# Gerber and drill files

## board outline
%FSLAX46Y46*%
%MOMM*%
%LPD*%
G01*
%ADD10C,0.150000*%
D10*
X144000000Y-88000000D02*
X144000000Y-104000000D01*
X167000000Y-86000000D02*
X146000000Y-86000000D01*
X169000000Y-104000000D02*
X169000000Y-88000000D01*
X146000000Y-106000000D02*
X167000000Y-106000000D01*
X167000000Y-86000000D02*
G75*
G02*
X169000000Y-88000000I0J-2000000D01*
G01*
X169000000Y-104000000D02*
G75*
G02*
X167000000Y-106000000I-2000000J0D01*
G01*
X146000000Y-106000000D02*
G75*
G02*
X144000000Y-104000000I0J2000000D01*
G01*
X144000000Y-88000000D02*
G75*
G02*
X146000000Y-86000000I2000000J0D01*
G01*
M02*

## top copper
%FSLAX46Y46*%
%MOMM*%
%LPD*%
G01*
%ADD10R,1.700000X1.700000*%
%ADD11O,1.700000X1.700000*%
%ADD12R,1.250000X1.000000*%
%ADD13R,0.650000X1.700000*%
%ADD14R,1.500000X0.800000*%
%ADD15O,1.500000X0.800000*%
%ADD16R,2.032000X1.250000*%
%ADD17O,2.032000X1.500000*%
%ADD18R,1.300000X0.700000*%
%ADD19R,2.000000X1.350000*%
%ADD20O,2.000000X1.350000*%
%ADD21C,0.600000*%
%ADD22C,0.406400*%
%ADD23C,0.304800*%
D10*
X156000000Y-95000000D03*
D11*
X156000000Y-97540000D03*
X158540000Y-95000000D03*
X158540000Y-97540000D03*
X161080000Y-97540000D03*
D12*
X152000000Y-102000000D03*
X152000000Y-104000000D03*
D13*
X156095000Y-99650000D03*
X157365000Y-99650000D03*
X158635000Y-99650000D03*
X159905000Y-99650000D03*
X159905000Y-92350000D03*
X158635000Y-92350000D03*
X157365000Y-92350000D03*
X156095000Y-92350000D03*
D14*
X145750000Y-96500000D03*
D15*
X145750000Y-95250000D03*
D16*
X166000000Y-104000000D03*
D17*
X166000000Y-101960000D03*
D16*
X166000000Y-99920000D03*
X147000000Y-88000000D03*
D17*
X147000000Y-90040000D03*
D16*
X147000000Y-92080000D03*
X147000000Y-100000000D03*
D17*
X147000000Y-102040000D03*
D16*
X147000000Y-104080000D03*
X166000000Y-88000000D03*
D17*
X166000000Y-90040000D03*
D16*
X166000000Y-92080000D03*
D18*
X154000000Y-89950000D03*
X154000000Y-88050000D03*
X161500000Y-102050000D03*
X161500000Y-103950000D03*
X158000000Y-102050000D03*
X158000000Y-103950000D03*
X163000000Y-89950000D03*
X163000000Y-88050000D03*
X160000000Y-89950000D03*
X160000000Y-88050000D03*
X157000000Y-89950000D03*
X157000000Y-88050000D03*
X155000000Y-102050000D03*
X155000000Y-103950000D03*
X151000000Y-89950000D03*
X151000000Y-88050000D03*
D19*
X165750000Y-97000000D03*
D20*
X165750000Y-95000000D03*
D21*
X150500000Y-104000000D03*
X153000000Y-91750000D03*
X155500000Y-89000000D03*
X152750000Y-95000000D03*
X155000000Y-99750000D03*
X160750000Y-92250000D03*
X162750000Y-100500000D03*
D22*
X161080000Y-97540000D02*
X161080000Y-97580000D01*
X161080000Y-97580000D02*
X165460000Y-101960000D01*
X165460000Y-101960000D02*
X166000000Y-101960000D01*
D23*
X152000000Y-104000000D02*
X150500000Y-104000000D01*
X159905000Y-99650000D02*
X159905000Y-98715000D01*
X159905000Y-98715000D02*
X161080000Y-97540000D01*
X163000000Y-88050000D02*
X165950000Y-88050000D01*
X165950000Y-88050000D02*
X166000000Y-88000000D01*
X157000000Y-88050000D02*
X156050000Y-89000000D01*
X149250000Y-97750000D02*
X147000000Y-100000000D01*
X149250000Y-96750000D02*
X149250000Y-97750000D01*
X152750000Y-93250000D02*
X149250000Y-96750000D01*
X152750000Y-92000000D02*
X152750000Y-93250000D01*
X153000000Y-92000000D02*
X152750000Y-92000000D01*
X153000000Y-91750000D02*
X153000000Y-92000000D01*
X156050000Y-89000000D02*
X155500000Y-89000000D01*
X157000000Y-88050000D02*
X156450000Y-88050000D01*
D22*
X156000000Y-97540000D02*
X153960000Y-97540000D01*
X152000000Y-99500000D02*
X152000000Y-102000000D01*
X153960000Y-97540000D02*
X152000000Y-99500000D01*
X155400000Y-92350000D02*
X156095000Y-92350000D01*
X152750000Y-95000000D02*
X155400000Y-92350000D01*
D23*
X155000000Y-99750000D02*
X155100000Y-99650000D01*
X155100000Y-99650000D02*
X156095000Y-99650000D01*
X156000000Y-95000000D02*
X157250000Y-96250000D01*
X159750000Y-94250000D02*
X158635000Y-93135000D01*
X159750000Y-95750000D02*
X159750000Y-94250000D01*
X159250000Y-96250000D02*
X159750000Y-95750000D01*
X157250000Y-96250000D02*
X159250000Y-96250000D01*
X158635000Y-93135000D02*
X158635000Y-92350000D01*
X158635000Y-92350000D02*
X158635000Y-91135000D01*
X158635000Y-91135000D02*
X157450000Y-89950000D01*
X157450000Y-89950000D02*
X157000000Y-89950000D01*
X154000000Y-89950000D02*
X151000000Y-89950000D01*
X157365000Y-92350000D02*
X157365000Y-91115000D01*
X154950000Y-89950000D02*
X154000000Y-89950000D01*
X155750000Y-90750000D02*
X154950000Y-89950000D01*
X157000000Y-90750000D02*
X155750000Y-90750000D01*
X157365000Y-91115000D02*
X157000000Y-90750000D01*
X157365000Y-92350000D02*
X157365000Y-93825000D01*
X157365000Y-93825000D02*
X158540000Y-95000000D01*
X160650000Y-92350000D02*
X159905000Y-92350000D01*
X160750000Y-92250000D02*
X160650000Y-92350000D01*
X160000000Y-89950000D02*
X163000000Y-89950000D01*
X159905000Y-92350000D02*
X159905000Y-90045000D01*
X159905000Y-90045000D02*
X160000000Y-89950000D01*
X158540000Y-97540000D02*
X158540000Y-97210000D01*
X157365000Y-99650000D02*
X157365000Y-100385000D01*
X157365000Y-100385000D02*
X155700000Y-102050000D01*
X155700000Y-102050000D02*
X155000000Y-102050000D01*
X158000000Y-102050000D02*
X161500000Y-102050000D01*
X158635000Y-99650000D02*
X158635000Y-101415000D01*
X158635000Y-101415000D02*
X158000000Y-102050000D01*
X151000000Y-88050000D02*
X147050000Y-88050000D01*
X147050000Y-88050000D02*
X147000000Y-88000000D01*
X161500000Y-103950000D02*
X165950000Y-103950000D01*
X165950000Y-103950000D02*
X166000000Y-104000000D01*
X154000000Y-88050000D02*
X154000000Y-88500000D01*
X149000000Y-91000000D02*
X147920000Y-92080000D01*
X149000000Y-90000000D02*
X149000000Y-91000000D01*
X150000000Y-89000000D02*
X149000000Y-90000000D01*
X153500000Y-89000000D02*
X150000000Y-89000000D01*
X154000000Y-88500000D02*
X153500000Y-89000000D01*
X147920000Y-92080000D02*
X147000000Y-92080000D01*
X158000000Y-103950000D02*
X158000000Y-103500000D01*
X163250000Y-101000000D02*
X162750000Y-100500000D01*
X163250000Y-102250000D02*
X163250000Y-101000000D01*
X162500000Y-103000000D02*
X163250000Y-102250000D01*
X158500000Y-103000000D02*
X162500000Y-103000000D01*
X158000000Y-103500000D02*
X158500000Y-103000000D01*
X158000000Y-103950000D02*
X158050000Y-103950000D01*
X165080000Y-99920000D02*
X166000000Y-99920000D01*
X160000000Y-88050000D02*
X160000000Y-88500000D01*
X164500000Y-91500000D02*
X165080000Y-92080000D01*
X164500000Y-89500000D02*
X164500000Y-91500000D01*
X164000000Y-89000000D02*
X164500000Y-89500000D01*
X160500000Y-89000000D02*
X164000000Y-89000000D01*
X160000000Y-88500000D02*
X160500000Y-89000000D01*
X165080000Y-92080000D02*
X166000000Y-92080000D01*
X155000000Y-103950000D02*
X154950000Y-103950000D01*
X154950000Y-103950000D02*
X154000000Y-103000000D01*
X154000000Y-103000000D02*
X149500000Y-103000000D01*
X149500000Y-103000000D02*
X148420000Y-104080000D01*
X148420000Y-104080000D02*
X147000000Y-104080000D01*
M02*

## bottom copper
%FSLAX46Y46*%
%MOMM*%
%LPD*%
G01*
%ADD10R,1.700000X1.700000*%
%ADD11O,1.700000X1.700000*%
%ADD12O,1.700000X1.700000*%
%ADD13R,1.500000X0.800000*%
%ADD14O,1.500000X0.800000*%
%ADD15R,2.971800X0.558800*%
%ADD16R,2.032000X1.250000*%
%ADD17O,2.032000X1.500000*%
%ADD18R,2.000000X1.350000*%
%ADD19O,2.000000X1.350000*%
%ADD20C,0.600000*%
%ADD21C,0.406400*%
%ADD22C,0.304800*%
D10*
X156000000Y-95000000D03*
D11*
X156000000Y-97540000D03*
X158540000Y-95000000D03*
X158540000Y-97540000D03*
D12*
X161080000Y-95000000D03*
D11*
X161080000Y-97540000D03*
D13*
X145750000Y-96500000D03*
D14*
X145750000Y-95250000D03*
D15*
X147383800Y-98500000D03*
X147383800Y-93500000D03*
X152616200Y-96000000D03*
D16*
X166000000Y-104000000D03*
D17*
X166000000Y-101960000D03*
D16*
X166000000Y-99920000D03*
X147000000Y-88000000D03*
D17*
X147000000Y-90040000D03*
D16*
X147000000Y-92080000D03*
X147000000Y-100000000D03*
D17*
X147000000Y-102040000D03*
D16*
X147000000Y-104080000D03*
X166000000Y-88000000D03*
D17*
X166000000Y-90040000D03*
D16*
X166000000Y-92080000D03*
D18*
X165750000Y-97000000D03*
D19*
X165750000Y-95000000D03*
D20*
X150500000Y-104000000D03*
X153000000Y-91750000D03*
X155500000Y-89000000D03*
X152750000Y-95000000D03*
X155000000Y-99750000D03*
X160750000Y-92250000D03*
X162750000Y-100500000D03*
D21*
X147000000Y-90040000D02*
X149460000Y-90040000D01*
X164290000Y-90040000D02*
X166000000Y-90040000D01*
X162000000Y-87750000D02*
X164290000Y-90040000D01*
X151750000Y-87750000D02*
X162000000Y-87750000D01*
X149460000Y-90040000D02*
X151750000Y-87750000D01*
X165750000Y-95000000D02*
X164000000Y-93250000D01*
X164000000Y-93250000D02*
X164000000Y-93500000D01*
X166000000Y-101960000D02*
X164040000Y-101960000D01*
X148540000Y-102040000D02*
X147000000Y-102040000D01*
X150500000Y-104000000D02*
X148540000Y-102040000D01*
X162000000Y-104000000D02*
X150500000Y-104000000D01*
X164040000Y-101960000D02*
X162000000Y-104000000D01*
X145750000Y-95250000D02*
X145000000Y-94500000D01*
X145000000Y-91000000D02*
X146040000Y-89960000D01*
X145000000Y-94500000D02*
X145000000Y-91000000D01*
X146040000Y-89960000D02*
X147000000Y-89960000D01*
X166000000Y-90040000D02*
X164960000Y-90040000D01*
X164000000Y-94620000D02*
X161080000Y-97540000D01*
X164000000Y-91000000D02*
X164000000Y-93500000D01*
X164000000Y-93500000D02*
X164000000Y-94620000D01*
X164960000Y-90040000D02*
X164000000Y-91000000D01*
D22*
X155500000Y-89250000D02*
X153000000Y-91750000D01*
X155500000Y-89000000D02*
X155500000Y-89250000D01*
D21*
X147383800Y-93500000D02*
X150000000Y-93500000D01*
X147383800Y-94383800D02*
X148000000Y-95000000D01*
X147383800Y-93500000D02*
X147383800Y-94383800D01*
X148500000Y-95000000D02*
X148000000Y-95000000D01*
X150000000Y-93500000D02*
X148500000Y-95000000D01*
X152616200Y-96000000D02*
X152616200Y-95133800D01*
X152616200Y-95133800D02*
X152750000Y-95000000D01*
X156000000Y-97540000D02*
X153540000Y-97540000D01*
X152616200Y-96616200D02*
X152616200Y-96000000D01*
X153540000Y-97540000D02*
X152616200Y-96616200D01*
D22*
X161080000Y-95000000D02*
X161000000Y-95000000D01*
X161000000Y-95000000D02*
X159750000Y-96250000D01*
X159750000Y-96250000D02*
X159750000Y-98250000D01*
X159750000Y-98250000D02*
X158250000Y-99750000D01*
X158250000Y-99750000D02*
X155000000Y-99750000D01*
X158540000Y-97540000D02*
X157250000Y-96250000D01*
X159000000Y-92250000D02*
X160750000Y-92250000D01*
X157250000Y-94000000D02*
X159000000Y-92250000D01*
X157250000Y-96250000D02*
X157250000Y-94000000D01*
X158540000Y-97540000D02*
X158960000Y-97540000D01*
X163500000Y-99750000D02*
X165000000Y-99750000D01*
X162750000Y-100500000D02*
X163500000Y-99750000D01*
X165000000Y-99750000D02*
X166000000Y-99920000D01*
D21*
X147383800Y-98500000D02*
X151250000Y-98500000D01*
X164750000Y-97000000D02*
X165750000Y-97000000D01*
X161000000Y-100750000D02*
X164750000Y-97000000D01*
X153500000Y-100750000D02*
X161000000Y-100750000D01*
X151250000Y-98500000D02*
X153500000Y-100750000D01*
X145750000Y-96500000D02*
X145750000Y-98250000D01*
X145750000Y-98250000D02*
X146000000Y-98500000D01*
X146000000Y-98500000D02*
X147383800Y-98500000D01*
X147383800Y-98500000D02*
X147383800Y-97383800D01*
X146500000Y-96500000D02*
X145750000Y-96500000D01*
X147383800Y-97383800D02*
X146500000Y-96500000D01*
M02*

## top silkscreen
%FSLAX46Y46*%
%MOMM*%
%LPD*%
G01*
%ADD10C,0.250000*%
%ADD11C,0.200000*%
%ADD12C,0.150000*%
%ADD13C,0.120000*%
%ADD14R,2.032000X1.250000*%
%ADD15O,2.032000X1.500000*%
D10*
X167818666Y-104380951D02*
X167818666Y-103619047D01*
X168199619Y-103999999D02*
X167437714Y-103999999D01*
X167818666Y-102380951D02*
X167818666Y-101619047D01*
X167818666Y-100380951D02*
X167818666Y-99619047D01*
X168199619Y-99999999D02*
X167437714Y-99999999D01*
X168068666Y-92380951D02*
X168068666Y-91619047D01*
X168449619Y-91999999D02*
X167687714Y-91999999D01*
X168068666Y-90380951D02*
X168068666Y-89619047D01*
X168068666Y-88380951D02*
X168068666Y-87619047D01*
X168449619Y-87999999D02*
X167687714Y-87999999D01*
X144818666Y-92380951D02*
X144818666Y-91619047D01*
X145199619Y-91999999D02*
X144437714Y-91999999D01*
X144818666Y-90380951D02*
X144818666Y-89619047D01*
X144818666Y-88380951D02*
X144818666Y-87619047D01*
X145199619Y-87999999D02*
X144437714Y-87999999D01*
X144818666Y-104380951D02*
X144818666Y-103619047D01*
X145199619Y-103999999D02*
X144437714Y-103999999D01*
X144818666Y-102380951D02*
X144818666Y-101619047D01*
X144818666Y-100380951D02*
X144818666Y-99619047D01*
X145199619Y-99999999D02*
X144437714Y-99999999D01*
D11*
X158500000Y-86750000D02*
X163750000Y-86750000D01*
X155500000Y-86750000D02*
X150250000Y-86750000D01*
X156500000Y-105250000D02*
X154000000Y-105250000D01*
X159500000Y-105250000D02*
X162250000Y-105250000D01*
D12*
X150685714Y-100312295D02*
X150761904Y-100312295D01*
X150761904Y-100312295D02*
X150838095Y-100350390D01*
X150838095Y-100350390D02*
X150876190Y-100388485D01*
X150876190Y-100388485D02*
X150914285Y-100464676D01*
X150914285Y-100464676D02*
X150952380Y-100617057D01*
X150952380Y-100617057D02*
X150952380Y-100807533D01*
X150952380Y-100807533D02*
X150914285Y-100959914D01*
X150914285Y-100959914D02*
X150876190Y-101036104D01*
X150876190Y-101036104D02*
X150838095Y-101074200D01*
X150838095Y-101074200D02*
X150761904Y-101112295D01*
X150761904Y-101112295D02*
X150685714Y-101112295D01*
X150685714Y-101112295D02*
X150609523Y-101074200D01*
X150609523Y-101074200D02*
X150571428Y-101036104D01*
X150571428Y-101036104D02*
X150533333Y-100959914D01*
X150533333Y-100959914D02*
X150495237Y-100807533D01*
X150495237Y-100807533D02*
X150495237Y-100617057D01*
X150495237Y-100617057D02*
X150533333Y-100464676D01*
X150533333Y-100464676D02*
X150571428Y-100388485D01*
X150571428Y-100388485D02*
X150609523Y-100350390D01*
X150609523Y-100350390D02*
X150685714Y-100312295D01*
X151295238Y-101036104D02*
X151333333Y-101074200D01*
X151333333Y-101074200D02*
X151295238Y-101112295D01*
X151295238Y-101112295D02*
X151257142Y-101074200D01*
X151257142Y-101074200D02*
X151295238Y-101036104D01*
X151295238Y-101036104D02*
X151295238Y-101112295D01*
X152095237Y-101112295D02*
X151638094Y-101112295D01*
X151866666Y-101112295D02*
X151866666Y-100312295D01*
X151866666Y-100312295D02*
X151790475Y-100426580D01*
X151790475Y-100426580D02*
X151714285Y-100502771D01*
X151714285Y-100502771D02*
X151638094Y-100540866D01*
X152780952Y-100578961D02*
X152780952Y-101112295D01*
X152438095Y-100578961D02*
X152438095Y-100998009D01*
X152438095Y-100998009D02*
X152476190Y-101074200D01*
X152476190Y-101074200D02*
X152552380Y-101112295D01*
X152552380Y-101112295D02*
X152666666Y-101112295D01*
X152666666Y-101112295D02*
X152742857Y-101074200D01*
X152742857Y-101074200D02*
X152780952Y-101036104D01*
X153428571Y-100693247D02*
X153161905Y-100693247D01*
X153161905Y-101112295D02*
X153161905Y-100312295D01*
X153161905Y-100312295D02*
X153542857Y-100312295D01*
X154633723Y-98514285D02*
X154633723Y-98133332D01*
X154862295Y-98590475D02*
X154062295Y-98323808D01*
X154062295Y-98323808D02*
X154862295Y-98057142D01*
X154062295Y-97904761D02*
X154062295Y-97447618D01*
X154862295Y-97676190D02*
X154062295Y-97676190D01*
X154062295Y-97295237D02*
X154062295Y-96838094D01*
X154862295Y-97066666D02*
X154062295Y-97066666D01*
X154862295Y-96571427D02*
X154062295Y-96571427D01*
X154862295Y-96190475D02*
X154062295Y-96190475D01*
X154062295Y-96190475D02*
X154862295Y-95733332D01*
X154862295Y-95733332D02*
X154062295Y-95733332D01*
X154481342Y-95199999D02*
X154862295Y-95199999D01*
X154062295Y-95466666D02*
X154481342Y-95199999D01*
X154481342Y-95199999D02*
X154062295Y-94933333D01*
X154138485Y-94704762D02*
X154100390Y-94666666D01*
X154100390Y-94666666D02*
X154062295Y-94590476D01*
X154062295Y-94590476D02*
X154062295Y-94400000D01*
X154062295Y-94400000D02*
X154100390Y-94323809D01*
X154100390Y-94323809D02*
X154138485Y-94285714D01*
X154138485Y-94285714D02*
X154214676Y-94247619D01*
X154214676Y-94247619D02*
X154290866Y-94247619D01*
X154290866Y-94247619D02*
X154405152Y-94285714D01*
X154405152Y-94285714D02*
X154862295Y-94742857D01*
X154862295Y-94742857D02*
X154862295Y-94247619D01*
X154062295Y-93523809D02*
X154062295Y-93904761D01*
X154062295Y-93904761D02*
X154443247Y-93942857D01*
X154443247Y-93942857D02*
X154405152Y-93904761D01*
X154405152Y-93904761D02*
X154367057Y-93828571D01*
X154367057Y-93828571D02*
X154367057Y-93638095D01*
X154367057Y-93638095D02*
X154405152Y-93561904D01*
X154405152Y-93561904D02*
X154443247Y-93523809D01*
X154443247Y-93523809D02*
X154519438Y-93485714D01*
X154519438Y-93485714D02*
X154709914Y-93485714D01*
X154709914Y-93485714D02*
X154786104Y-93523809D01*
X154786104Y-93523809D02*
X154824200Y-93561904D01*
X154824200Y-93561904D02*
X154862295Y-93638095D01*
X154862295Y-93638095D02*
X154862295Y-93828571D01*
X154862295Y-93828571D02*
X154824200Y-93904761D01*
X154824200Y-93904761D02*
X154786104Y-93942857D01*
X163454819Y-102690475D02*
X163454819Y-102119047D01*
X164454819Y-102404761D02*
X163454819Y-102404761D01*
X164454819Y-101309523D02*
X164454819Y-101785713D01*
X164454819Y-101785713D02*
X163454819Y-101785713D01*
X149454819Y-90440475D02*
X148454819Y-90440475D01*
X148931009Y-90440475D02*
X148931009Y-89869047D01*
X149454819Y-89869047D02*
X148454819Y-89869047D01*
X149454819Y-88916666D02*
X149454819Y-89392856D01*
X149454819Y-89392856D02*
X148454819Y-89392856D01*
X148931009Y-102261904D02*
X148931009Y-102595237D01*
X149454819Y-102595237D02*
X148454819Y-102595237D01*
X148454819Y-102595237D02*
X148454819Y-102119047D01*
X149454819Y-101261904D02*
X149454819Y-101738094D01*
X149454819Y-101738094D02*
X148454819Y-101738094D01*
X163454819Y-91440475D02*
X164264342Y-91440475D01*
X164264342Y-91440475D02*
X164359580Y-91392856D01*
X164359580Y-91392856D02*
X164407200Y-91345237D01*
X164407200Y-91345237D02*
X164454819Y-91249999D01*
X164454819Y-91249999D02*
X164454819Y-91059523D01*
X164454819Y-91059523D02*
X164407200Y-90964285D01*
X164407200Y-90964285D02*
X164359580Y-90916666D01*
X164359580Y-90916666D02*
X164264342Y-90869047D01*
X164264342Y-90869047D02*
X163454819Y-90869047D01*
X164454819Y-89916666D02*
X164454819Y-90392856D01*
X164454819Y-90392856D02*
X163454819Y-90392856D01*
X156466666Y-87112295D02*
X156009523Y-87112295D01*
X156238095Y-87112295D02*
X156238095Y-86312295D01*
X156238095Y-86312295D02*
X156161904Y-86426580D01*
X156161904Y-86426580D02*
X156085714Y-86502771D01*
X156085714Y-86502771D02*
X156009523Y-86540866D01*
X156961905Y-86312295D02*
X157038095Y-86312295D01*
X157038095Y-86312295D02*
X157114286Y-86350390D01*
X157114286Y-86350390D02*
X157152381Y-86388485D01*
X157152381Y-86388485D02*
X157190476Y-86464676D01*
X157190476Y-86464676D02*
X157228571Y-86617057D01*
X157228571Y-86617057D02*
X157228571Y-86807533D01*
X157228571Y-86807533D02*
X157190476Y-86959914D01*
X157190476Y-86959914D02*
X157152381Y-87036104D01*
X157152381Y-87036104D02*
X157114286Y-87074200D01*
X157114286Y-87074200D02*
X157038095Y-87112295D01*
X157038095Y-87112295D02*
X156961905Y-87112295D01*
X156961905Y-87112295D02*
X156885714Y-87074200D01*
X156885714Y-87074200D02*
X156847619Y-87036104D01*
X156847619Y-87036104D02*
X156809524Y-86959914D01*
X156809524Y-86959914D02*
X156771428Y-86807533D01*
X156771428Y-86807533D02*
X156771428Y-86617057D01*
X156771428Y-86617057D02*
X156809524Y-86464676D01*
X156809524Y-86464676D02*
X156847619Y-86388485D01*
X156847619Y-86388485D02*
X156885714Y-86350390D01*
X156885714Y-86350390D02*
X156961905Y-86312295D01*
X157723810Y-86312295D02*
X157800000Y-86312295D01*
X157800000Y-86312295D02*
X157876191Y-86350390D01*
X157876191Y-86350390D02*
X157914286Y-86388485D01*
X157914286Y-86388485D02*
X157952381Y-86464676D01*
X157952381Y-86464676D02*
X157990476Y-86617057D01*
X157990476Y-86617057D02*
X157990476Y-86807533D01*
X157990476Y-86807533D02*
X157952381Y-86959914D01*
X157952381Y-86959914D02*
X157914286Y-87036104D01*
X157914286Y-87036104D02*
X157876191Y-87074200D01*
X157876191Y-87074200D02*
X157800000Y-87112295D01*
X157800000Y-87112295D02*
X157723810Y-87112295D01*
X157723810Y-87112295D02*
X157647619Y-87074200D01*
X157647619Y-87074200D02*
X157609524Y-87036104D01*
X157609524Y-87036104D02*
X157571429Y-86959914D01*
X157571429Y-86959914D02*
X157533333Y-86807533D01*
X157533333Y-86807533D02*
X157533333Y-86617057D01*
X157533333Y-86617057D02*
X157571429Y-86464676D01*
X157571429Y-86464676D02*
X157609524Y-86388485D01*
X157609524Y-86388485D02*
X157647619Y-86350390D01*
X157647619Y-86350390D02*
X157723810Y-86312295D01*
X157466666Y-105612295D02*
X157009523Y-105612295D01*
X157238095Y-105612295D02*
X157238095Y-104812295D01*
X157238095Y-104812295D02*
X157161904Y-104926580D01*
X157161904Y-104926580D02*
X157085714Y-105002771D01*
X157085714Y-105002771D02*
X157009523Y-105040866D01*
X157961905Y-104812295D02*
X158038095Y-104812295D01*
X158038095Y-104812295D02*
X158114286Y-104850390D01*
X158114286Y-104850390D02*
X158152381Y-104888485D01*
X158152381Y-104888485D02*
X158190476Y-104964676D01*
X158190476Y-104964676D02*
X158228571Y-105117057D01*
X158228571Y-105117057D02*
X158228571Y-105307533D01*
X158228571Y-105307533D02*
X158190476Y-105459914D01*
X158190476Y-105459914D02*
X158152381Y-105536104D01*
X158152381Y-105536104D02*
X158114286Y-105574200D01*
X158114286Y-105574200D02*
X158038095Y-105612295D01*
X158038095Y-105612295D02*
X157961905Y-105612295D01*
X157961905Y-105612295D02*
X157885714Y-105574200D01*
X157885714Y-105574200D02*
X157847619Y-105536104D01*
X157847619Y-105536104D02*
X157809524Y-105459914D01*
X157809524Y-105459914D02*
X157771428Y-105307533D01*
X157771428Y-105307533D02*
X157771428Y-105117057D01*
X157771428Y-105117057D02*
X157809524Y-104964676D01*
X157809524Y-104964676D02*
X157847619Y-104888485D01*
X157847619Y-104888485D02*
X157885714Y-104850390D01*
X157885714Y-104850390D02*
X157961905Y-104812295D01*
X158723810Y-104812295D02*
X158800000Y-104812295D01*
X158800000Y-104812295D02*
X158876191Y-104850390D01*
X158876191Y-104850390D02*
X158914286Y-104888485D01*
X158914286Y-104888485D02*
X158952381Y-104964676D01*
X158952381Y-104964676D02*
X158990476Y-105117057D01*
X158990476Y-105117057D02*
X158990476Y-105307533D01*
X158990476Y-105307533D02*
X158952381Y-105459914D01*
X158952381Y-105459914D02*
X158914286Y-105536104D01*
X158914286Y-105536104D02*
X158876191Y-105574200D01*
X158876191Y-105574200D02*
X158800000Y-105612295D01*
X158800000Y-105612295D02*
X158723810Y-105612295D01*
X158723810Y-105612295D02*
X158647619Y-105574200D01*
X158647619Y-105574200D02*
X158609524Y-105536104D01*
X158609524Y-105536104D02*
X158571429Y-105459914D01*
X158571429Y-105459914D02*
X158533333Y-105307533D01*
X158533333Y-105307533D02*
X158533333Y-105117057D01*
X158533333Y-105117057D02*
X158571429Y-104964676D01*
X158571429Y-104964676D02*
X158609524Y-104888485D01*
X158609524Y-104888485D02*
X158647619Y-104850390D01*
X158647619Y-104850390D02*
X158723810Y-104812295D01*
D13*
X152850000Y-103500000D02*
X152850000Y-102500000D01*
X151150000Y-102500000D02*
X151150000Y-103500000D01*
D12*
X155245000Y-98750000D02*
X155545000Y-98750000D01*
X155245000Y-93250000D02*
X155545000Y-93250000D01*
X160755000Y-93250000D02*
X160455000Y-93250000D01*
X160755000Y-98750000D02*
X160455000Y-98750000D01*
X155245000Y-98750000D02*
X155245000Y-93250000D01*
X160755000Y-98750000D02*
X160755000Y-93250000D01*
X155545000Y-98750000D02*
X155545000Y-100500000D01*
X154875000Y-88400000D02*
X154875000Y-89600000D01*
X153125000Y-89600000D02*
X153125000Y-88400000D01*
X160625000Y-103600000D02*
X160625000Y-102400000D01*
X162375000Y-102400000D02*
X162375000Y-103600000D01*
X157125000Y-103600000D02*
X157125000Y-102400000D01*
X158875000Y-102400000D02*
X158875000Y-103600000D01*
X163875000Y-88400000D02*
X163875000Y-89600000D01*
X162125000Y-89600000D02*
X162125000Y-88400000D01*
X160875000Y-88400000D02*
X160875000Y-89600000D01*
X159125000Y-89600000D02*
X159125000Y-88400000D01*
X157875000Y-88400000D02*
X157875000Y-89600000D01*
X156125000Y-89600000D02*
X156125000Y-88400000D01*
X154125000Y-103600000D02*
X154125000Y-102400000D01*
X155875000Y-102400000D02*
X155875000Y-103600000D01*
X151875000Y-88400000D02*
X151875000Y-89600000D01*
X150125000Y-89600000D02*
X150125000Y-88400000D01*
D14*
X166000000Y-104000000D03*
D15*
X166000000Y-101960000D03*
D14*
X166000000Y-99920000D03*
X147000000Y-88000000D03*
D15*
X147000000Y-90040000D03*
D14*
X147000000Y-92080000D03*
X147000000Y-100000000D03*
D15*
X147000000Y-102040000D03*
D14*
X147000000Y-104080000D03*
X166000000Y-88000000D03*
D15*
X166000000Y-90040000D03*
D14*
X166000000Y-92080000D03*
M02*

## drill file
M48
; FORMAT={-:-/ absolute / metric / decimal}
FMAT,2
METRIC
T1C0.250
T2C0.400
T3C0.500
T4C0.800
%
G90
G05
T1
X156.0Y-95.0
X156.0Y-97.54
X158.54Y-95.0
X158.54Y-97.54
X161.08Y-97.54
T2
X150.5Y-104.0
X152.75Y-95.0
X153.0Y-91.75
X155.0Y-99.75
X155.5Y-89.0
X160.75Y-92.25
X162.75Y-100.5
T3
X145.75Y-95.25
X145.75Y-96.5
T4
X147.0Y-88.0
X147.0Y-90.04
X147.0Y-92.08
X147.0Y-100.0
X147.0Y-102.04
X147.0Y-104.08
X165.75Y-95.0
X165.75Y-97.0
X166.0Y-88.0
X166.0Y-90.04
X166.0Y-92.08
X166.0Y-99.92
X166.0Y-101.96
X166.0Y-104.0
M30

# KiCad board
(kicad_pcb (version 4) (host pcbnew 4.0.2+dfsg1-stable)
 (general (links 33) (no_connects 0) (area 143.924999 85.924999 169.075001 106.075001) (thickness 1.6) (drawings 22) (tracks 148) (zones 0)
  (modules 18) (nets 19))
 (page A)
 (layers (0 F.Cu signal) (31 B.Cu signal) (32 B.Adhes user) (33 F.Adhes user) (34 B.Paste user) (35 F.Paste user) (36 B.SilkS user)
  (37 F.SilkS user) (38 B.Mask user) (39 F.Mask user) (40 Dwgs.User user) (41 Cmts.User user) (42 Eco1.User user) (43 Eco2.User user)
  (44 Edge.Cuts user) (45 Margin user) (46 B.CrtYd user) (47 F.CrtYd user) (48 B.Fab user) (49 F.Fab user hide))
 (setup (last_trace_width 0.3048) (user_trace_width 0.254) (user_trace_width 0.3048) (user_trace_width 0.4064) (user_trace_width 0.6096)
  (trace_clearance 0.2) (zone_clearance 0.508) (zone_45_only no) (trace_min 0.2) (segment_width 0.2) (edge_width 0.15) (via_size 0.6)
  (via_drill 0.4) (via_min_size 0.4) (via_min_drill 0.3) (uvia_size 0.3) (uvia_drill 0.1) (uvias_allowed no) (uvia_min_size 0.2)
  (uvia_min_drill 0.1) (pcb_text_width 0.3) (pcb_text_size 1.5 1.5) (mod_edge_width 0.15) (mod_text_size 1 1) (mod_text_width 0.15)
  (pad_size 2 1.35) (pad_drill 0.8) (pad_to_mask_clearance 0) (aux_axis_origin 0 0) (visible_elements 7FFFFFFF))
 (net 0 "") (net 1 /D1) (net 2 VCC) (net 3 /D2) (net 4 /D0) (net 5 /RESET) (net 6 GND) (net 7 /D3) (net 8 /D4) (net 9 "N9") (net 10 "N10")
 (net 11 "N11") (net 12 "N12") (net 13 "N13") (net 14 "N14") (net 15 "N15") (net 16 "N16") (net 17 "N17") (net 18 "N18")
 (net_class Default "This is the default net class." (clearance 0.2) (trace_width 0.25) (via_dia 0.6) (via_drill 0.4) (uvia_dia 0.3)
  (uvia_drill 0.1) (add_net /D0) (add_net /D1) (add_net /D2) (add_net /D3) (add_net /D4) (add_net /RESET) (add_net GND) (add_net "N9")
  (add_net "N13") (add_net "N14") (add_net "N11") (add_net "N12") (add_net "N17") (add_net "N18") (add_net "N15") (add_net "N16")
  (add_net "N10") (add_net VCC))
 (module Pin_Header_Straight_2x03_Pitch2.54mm (layer B.Cu) (at 156 95 270)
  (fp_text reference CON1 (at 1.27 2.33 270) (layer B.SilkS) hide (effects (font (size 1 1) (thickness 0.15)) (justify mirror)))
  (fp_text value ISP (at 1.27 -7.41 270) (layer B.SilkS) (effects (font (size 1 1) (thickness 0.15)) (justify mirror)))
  (pad 1 thru_hole rect (at 0 0 270) (size 1.7 1.7) (drill 0.25) (layers *.Cu *.Mask B.SilkS) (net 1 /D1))
  (pad 2 thru_hole oval (at 2.54 0 270) (size 1.7 1.7) (drill 0.25) (layers *.Cu *.Mask B.SilkS) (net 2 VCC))
  (pad 3 thru_hole oval (at 0 -2.54 270) (size 1.7 1.7) (drill 0.25) (layers *.Cu *.Mask B.SilkS) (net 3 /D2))
  (pad 4 thru_hole oval (at 2.54 -2.54 270) (size 1.7 1.7) (drill 0.25) (layers *.Cu *.Mask B.SilkS) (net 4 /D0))
  (pad 5 smd oval (at 0 -5.08 270) (size 1.7 1.7) (layers B.Cu B.Paste B.Mask) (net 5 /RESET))
  (pad 6 thru_hole oval (at 2.54 -5.08 270) (size 1.7 1.7) (drill 0.25) (layers *.Cu *.Mask B.SilkS) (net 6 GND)))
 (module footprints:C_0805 (layer F.Cu) (at 152 103 270)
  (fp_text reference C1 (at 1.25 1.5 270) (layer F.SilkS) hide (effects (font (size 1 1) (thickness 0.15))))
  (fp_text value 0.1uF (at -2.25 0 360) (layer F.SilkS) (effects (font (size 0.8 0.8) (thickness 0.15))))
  (fp_line (start 0.5 -0.85) (end -0.5 -0.85) (layer F.SilkS) (width 0.12))
  (fp_line (start -0.5 0.85) (end 0.5 0.85) (layer F.SilkS) (width 0.12))
  (pad 1 smd rect (at -1 0 270) (size 1 1.25) (layers F.Cu F.Paste F.Mask) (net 2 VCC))
  (pad 2 smd rect (at 1 0 270) (size 1 1.25) (layers F.Cu F.Paste F.Mask) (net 6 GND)))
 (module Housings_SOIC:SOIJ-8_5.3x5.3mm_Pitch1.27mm (layer F.Cu) (at 158 96 90)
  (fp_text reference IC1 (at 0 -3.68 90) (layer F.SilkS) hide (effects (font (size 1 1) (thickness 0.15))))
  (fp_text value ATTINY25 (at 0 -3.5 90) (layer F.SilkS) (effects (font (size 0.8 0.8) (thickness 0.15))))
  (fp_line (start -2.75 -2.755) (end -2.75 -2.455) (layer F.SilkS) (width 0.15))
  (fp_line (start 2.75 -2.755) (end 2.75 -2.455) (layer F.SilkS) (width 0.15))
  (fp_line (start 2.75 2.755) (end 2.75 2.455) (layer F.SilkS) (width 0.15))
  (fp_line (start -2.75 2.755) (end -2.75 2.455) (layer F.SilkS) (width 0.15))
  (fp_line (start -2.75 -2.755) (end 2.75 -2.755) (layer F.SilkS) (width 0.15))
  (fp_line (start -2.75 2.755) (end 2.75 2.755) (layer F.SilkS) (width 0.15))
  (fp_line (start -2.75 -2.455) (end -4.5 -2.455) (layer F.SilkS) (width 0.15))
  (pad 1 smd rect (at -3.65 -1.905 90) (size 1.7 0.65) (layers F.Cu F.Paste F.Mask) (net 5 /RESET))
  (pad 2 smd rect (at -3.65 -0.635 90) (size 1.7 0.65) (layers F.Cu F.Paste F.Mask) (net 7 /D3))
  (pad 3 smd rect (at -3.65 0.635 90) (size 1.7 0.65) (layers F.Cu F.Paste F.Mask) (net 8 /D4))
  (pad 4 smd rect (at -3.65 1.905 90) (size 1.7 0.65) (layers F.Cu F.Paste F.Mask) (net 6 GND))
  (pad 5 smd rect (at 3.65 1.905 90) (size 1.7 0.65) (layers F.Cu F.Paste F.Mask) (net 4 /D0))
  (pad 6 smd rect (at 3.65 0.635 90) (size 1.7 0.65) (layers F.Cu F.Paste F.Mask) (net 1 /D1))
  (pad 7 smd rect (at 3.65 -0.635 90) (size 1.7 0.65) (layers F.Cu F.Paste F.Mask) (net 3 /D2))
  (pad 8 smd rect (at 3.65 -1.905 90) (size 1.7 0.65) (layers F.Cu F.Paste F.Mask) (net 2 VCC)))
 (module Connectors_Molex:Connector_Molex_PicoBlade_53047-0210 (layer B.Cu) (at 145.75 96.5 90)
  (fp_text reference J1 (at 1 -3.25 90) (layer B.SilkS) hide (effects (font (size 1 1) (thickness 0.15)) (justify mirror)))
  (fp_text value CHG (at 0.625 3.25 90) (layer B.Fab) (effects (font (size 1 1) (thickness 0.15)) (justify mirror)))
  (pad 1 thru_hole rect (at 0 0 90) (size 0.8 1.5) (drill 0.5) (layers *.Cu *.Mask B.SilkS) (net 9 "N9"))
  (pad 2 thru_hole oval (at 1.25 0 90) (size 0.8 1.5) (drill 0.5) (layers *.Cu *.Mask B.SilkS) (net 6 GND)))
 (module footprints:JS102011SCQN (layer B.Cu) (at 150 96)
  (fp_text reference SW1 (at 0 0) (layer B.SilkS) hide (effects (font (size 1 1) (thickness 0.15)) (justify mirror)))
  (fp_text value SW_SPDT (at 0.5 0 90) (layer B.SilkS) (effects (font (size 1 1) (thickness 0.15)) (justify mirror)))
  (pad 1 smd rect (at -2.6162 2.5) (size 2.9718 0.5588) (layers B.Cu B.Paste B.Mask) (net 9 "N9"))
  (pad 3 smd rect (at -2.6162 -2.5) (size 2.9718 0.5588) (layers B.Cu B.Paste B.Mask) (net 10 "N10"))
  (pad 2 smd rect (at 2.6162 0) (size 2.9718 0.5588) (layers B.Cu B.Paste B.Mask) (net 2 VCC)))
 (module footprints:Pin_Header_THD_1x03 (layer F.Cu) (at 166 104 180)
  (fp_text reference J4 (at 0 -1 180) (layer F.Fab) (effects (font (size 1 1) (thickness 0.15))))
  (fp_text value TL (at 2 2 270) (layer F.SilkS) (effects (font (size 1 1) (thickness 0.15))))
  (pad 1 thru_hole rect (at 0 0 180) (size 2.032 1.25) (drill 0.8) (layers *.Cu *.Mask F.SilkS) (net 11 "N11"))
  (pad 2 thru_hole oval (at 0 2.04 180) (size 2.032 1.5) (drill 0.8) (layers *.Cu *.Mask F.SilkS) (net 6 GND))
  (pad 3 thru_hole rect (at 0 4.08 180) (size 2.032 1.25) (drill 0.8) (layers *.Cu *.Mask F.SilkS) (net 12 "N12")))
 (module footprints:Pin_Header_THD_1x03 (layer F.Cu) (at 147 88)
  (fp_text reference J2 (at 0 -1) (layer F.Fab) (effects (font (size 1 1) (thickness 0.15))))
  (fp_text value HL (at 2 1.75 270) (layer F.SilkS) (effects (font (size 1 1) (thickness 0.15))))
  (pad 1 thru_hole rect (at 0 0) (size 2.032 1.25) (drill 0.8) (layers *.Cu *.Mask F.SilkS) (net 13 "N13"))
  (pad 2 thru_hole oval (at 0 2.04) (size 2.032 1.5) (drill 0.8) (layers *.Cu *.Mask F.SilkS) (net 6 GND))
  (pad 3 thru_hole rect (at 0 4.08) (size 2.032 1.25) (drill 0.8) (layers *.Cu *.Mask F.SilkS) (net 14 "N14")))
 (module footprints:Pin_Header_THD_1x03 (layer F.Cu) (at 147 100)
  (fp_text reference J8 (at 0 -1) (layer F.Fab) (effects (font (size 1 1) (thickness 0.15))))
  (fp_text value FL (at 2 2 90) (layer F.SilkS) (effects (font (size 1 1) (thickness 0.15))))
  (pad 1 thru_hole rect (at 0 0) (size 2.032 1.25) (drill 0.8) (layers *.Cu *.Mask F.SilkS) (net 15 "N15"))
  (pad 2 thru_hole oval (at 0 2.04) (size 2.032 1.5) (drill 0.8) (layers *.Cu *.Mask F.SilkS) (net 6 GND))
  (pad 3 thru_hole rect (at 0 4.08) (size 2.032 1.25) (drill 0.8) (layers *.Cu *.Mask F.SilkS) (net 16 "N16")))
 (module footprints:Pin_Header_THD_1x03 (layer F.Cu) (at 166 88)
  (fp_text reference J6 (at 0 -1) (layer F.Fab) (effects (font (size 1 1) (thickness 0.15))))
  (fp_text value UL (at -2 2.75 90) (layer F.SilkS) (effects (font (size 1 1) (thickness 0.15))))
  (pad 1 thru_hole rect (at 0 0) (size 2.032 1.25) (drill 0.8) (layers *.Cu *.Mask F.SilkS) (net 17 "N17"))
  (pad 2 thru_hole oval (at 0 2.04) (size 2.032 1.5) (drill 0.8) (layers *.Cu *.Mask F.SilkS) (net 6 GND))
  (pad 3 thru_hole rect (at 0 4.08) (size 2.032 1.25) (drill 0.8) (layers *.Cu *.Mask F.SilkS) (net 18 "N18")))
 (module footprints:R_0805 (layer F.Cu) (at 154 89 90)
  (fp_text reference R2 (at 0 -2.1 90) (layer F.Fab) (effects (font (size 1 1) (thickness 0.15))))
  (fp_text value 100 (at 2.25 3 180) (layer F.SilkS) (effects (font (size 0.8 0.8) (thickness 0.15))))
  (fp_line (start 0.6 0.875) (end -0.6 0.875) (layer F.SilkS) (width 0.15))
  (fp_line (start -0.6 -0.875) (end 0.6 -0.875) (layer F.SilkS) (width 0.15))
  (pad 1 smd rect (at -0.95 0 90) (size 0.7 1.3) (layers F.Cu F.Paste F.Mask) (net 3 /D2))
  (pad 2 smd rect (at 0.95 0 90) (size 0.7 1.3) (layers F.Cu F.Paste F.Mask) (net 14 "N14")))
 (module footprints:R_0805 (layer F.Cu) (at 161.5 103 270)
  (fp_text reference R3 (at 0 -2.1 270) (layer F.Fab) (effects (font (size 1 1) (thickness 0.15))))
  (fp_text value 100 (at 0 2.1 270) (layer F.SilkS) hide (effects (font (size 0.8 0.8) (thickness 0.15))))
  (fp_line (start 0.6 0.875) (end -0.6 0.875) (layer F.SilkS) (width 0.15))
  (fp_line (start -0.6 -0.875) (end 0.6 -0.875) (layer F.SilkS) (width 0.15))
  (pad 1 smd rect (at -0.95 0 270) (size 0.7 1.3) (layers F.Cu F.Paste F.Mask) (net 8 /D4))
  (pad 2 smd rect (at 0.95 0 270) (size 0.7 1.3) (layers F.Cu F.Paste F.Mask) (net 11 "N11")))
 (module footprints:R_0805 (layer F.Cu) (at 158 103 270)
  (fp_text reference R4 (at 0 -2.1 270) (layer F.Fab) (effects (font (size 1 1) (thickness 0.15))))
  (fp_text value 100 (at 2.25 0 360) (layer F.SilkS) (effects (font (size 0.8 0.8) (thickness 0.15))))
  (fp_line (start 0.6 0.875) (end -0.6 0.875) (layer F.SilkS) (width 0.15))
  (fp_line (start -0.6 -0.875) (end 0.6 -0.875) (layer F.SilkS) (width 0.15))
  (pad 1 smd rect (at -0.95 0 270) (size 0.7 1.3) (layers F.Cu F.Paste F.Mask) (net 8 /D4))
  (pad 2 smd rect (at 0.95 0 270) (size 0.7 1.3) (layers F.Cu F.Paste F.Mask) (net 12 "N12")))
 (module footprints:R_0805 (layer F.Cu) (at 163 89 90)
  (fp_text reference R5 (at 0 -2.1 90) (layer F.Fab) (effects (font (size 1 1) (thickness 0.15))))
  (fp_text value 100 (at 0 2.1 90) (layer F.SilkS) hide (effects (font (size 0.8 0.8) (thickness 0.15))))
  (fp_line (start 0.6 0.875) (end -0.6 0.875) (layer F.SilkS) (width 0.15))
  (fp_line (start -0.6 -0.875) (end 0.6 -0.875) (layer F.SilkS) (width 0.15))
  (pad 1 smd rect (at -0.95 0 90) (size 0.7 1.3) (layers F.Cu F.Paste F.Mask) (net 4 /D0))
  (pad 2 smd rect (at 0.95 0 90) (size 0.7 1.3) (layers F.Cu F.Paste F.Mask) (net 17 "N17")))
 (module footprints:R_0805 (layer F.Cu) (at 160 89 90)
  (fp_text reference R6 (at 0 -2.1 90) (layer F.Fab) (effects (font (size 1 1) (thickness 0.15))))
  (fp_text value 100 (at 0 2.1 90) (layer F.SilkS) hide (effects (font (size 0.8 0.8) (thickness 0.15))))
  (fp_line (start 0.6 0.875) (end -0.6 0.875) (layer F.SilkS) (width 0.15))
  (fp_line (start -0.6 -0.875) (end 0.6 -0.875) (layer F.SilkS) (width 0.15))
  (pad 1 smd rect (at -0.95 0 90) (size 0.7 1.3) (layers F.Cu F.Paste F.Mask) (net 4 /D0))
  (pad 2 smd rect (at 0.95 0 90) (size 0.7 1.3) (layers F.Cu F.Paste F.Mask) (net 18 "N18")))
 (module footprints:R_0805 (layer F.Cu) (at 157 89 90)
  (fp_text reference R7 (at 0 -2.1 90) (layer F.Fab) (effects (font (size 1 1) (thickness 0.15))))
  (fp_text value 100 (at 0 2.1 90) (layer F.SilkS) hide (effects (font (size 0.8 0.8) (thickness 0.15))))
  (fp_line (start 0.6 0.875) (end -0.6 0.875) (layer F.SilkS) (width 0.15))
  (fp_line (start -0.6 -0.875) (end 0.6 -0.875) (layer F.SilkS) (width 0.15))
  (pad 1 smd rect (at -0.95 0 90) (size 0.7 1.3) (layers F.Cu F.Paste F.Mask) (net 1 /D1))
  (pad 2 smd rect (at 0.95 0 90) (size 0.7 1.3) (layers F.Cu F.Paste F.Mask) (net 15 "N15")))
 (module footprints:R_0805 (layer F.Cu) (at 155 103 270)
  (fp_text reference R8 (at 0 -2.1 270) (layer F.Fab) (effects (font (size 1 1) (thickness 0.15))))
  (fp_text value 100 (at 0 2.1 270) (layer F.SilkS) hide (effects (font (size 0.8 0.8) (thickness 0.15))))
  (fp_line (start 0.6 0.875) (end -0.6 0.875) (layer F.SilkS) (width 0.15))
  (fp_line (start -0.6 -0.875) (end 0.6 -0.875) (layer F.SilkS) (width 0.15))
  (pad 1 smd rect (at -0.95 0 270) (size 0.7 1.3) (layers F.Cu F.Paste F.Mask) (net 7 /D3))
  (pad 2 smd rect (at 0.95 0 270) (size 0.7 1.3) (layers F.Cu F.Paste F.Mask) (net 16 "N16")))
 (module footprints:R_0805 (layer F.Cu) (at 151 89 90)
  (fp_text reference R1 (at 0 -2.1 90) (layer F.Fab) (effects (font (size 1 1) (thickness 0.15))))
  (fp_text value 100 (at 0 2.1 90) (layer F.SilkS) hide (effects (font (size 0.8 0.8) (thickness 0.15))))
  (fp_line (start 0.6 0.875) (end -0.6 0.875) (layer F.SilkS) (width 0.15))
  (fp_line (start -0.6 -0.875) (end 0.6 -0.875) (layer F.SilkS) (width 0.15))
  (pad 1 smd rect (at -0.95 0 90) (size 0.7 1.3) (layers F.Cu F.Paste F.Mask) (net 3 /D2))
  (pad 2 smd rect (at 0.95 0 90) (size 0.7 1.3) (layers F.Cu F.Paste F.Mask) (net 13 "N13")))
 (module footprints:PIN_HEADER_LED (layer B.Cu) (at 165.75 97)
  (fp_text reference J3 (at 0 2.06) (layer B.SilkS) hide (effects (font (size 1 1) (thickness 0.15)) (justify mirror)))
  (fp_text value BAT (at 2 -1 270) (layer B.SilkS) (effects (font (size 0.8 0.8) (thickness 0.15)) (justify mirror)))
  (pad 1 thru_hole rect (at 0 0) (size 2 1.35) (drill 0.8) (layers *.Cu *.Mask) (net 9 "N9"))
  (pad 2 thru_hole oval (at 0 -2) (size 2 1.35) (drill 0.8) (layers *.Cu *.Mask) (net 6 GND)))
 (gr_line (start 144 88) (end 144 104) (angle 90) (layer Edge.Cuts) (width 0.15))
 (gr_line (start 167 86) (end 146 86) (angle 90) (layer Edge.Cuts) (width 0.15))
 (gr_line (start 169 104) (end 169 88) (angle 90) (layer Edge.Cuts) (width 0.15))
 (gr_line (start 146 106) (end 167 106) (angle 90) (layer Edge.Cuts) (width 0.15))
 (gr_arc (start 167 88) (end 167 86) (angle 90) (layer Edge.Cuts) (width 0.15))
 (gr_arc (start 167 104) (end 169 104) (angle 90) (layer Edge.Cuts) (width 0.15))
 (gr_arc (start 146 104) (end 146 106) (angle 90) (layer Edge.Cuts) (width 0.15))
 (gr_arc (start 146 88) (end 144 88) (angle 90) (layer Edge.Cuts) (width 0.15))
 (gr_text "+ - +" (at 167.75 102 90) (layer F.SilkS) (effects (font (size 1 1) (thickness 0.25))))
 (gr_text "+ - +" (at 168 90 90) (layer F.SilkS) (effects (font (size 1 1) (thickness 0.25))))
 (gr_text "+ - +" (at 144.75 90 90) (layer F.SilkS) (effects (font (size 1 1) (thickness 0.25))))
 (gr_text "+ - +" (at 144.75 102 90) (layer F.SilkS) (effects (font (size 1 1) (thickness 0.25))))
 (gr_line (start 158.5 86.75) (end 163.75 86.75) (angle 90) (layer F.SilkS) (width 0.2))
 (gr_line (start 155.5 86.75) (end 150.25 86.75) (angle 90) (layer F.SilkS) (width 0.2))
 (gr_line (start 156.5 105.25) (end 154 105.25) (angle 90) (layer F.SilkS) (width 0.2))
 (gr_line (start 159.5 105.25) (end 162.25 105.25) (angle 90) (layer F.SilkS) (width 0.2))
 (segment (start 161.08 97.54) (end 161.08 97.58) (width 0.4064) (layer F.Cu) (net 6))
 (segment (start 161.08 97.58) (end 165.46 101.96) (width 0.4064) (layer F.Cu) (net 6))
 (segment (start 165.46 101.96) (end 166 101.96) (width 0.4064) (layer F.Cu) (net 6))
 (segment (start 147 90.04) (end 149.46 90.04) (width 0.4064) (layer B.Cu) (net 6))
 (segment (start 164.29 90.04) (end 166 90.04) (width 0.4064) (layer B.Cu) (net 6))
 (segment (start 162 87.75) (end 164.29 90.04) (width 0.4064) (layer B.Cu) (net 6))
 (segment (start 151.75 87.75) (end 162 87.75) (width 0.4064) (layer B.Cu) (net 6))
 (segment (start 149.46 90.04) (end 151.75 87.75) (width 0.4064) (layer B.Cu) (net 6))
 (segment (start 165.75 95) (end 164 93.25) (width 0.4064) (layer B.Cu) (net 6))
 (segment (start 164 93.25) (end 164 93.5) (width 0.4064) (layer B.Cu) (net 6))
 (segment (start 152 104) (end 150.5 104) (width 0.3048) (layer F.Cu) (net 6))
 (via (at 150.5 104) (size 0.6) (drill 0.4) (layers F.Cu B.Cu) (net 6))
 (segment (start 166 101.96) (end 164.04 101.96) (width 0.4064) (layer B.Cu) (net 6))
 (segment (start 148.54 102.04) (end 147 102.04) (width 0.4064) (layer B.Cu) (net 6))
 (segment (start 150.5 104) (end 148.54 102.04) (width 0.4064) (layer B.Cu) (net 6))
 (segment (start 162 104) (end 150.5 104) (width 0.4064) (layer B.Cu) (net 6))
 (segment (start 164.04 101.96) (end 162 104) (width 0.4064) (layer B.Cu) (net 6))
 (segment (start 145.75 95.25) (end 145 94.5) (width 0.4064) (layer B.Cu) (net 6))
 (segment (start 145 91) (end 146.04 89.96) (width 0.4064) (layer B.Cu) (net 6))
 (segment (start 145 94.5) (end 145 91) (width 0.4064) (layer B.Cu) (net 6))
 (segment (start 146.04 89.96) (end 147 89.96) (width 0.4064) (layer B.Cu) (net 6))
 (segment (start 166 90.04) (end 164.96 90.04) (width 0.4064) (layer B.Cu) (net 6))
 (segment (start 164 94.62) (end 161.08 97.54) (width 0.4064) (layer B.Cu) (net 6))
 (segment (start 164 91) (end 164 93.5) (width 0.4064) (layer B.Cu) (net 6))
 (segment (start 164 93.5) (end 164 94.62) (width 0.4064) (layer B.Cu) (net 6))
 (segment (start 164.96 90.04) (end 164 91) (width 0.4064) (layer B.Cu) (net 6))
 (segment (start 159.905 99.65) (end 159.905 98.715) (width 0.3048) (layer F.Cu) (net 6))
 (segment (start 159.905 98.715) (end 161.08 97.54) (width 0.3048) (layer F.Cu) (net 6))
 (segment (start 163 88.05) (end 165.95 88.05) (width 0.3048) (layer F.Cu) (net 17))
 (segment (start 165.95 88.05) (end 166 88) (width 0.3048) (layer F.Cu) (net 17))
 (segment (start 157 88.05) (end 156.05 89) (width 0.3048) (layer F.Cu) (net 15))
 (segment (start 149.25 97.75) (end 147 100) (width 0.3048) (layer F.Cu) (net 15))
 (segment (start 149.25 96.75) (end 149.25 97.75) (width 0.3048) (layer F.Cu) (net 15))
 (segment (start 152.75 93.25) (end 149.25 96.75) (width 0.3048) (layer F.Cu) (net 15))
 (segment (start 152.75 92) (end 152.75 93.25) (width 0.3048) (layer F.Cu) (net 15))
 (segment (start 153 92) (end 152.75 92) (width 0.3048) (layer F.Cu) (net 15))
 (segment (start 153 91.75) (end 153 92) (width 0.3048) (layer F.Cu) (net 15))
 (via (at 153 91.75) (size 0.6) (drill 0.4) (layers F.Cu B.Cu) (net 15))
 (segment (start 155.5 89.25) (end 153 91.75) (width 0.3048) (layer B.Cu) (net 15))
 (segment (start 155.5 89) (end 155.5 89.25) (width 0.3048) (layer B.Cu) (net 15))
 (via (at 155.5 89) (size 0.6) (drill 0.4) (layers F.Cu B.Cu) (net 15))
 (segment (start 156.05 89) (end 155.5 89) (width 0.3048) (layer F.Cu) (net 15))
 (segment (start 157 88.05) (end 156.45 88.05) (width 0.3048) (layer F.Cu) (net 15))
 (segment (start 147.3838 93.5) (end 150 93.5) (width 0.4064) (layer B.Cu) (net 10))
 (segment (start 147.3838 94.3838) (end 148 95) (width 0.4064) (layer B.Cu) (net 10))
 (segment (start 147.3838 93.5) (end 147.3838 94.3838) (width 0.4064) (layer B.Cu) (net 10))
 (segment (start 148.5 95) (end 148 95) (width 0.4064) (layer B.Cu) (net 10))
 (segment (start 150 93.5) (end 148.5 95) (width 0.4064) (layer B.Cu) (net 10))
 (segment (start 156 97.54) (end 153.96 97.54) (width 0.4064) (layer F.Cu) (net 2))
 (segment (start 152 99.5) (end 152 102) (width 0.4064) (layer F.Cu) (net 2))
 (segment (start 153.96 97.54) (end 152 99.5) (width 0.4064) (layer F.Cu) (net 2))
 (segment (start 152.6162 96) (end 152.6162 95.1338) (width 0.4064) (layer B.Cu) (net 2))
 (segment (start 155.4 92.35) (end 156.095 92.35) (width 0.4064) (layer F.Cu) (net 2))
 (segment (start 152.75 95) (end 155.4 92.35) (width 0.4064) (layer F.Cu) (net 2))
 (via (at 152.75 95) (size 0.6) (drill 0.4) (layers F.Cu B.Cu) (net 2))
 (segment (start 152.6162 95.1338) (end 152.75 95) (width 0.4064) (layer B.Cu) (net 2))
 (segment (start 156 97.54) (end 153.54 97.54) (width 0.4064) (layer B.Cu) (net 2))
 (segment (start 152.6162 96.6162) (end 152.6162 96) (width 0.4064) (layer B.Cu) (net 2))
 (segment (start 153.54 97.54) (end 152.6162 96.6162) (width 0.4064) (layer B.Cu) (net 2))
 (segment (start 161.08 95) (end 161 95) (width 0.3048) (layer B.Cu) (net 5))
 (segment (start 161 95) (end 159.75 96.25) (width 0.3048) (layer B.Cu) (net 5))
 (segment (start 159.75 96.25) (end 159.75 98.25) (width 0.3048) (layer B.Cu) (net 5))
 (segment (start 159.75 98.25) (end 158.25 99.75) (width 0.3048) (layer B.Cu) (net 5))
 (segment (start 158.25 99.75) (end 155 99.75) (width 0.3048) (layer B.Cu) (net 5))
 (via (at 155 99.75) (size 0.6) (drill 0.4) (layers F.Cu B.Cu) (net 5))
 (segment (start 155 99.75) (end 155.1 99.65) (width 0.3048) (layer F.Cu) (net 5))
 (segment (start 155.1 99.65) (end 156.095 99.65) (width 0.3048) (layer F.Cu) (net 5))
 (segment (start 156 95) (end 157.25 96.25) (width 0.3048) (layer F.Cu) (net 1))
 (segment (start 159.75 94.25) (end 158.635 93.135) (width 0.3048) (layer F.Cu) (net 1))
 (segment (start 159.75 95.75) (end 159.75 94.25) (width 0.3048) (layer F.Cu) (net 1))
 (segment (start 159.25 96.25) (end 159.75 95.75) (width 0.3048) (layer F.Cu) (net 1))
 (segment (start 157.25 96.25) (end 159.25 96.25) (width 0.3048) (layer F.Cu) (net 1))
 (segment (start 158.635 93.135) (end 158.635 92.35) (width 0.3048) (layer F.Cu) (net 1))
 (segment (start 158.635 92.35) (end 158.635 91.135) (width 0.3048) (layer F.Cu) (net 1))
 (segment (start 158.635 91.135) (end 157.45 89.95) (width 0.3048) (layer F.Cu) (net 1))
 (segment (start 157.45 89.95) (end 157 89.95) (width 0.3048) (layer F.Cu) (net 1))
 (segment (start 154 89.95) (end 151 89.95) (width 0.3048) (layer F.Cu) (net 3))
 (segment (start 157.365 92.35) (end 157.365 91.115) (width 0.3048) (layer F.Cu) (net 3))
 (segment (start 154.95 89.95) (end 154 89.95) (width 0.3048) (layer F.Cu) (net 3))
 (segment (start 155.75 90.75) (end 154.95 89.95) (width 0.3048) (layer F.Cu) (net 3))
 (segment (start 157 90.75) (end 155.75 90.75) (width 0.3048) (layer F.Cu) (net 3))
 (segment (start 157.365 91.115) (end 157 90.75) (width 0.3048) (layer F.Cu) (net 3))
 (segment (start 157.365 92.35) (end 157.365 93.825) (width 0.3048) (layer F.Cu) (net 3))
 (segment (start 157.365 93.825) (end 158.54 95) (width 0.3048) (layer F.Cu) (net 3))
 (segment (start 158.54 97.54) (end 157.25 96.25) (width 0.3048) (layer B.Cu) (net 4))
 (segment (start 159 92.25) (end 160.75 92.25) (width 0.3048) (layer B.Cu) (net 4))
 (segment (start 157.25 94) (end 159 92.25) (width 0.3048) (layer B.Cu) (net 4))
 (segment (start 157.25 96.25) (end 157.25 94) (width 0.3048) (layer B.Cu) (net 4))
 (segment (start 158.54 97.54) (end 158.96 97.54) (width 0.3048) (layer B.Cu) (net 4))
 (segment (start 160.65 92.35) (end 159.905 92.35) (width 0.3048) (layer F.Cu) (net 4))
 (via (at 160.75 92.25) (size 0.6) (drill 0.4) (layers F.Cu B.Cu) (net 4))
 (segment (start 160.75 92.25) (end 160.65 92.35) (width 0.3048) (layer F.Cu) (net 4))
 (segment (start 160 89.95) (end 163 89.95) (width 0.3048) (layer F.Cu) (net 4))
 (segment (start 159.905 92.35) (end 159.905 90.045) (width 0.3048) (layer F.Cu) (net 4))
 (segment (start 159.905 90.045) (end 160 89.95) (width 0.3048) (layer F.Cu) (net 4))
 (segment (start 158.54 97.54) (end 158.54 97.21) (width 0.3048) (layer F.Cu) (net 4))
 (segment (start 157.365 99.65) (end 157.365 100.385) (width 0.3048) (layer F.Cu) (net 7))
 (segment (start 157.365 100.385) (end 155.7 102.05) (width 0.3048) (layer F.Cu) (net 7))
 (segment (start 155.7 102.05) (end 155 102.05) (width 0.3048) (layer F.Cu) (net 7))
 (segment (start 158 102.05) (end 161.5 102.05) (width 0.3048) (layer F.Cu) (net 8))
 (segment (start 158.635 99.65) (end 158.635 101.415) (width 0.3048) (layer F.Cu) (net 8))
 (segment (start 158.635 101.415) (end 158 102.05) (width 0.3048) (layer F.Cu) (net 8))
 (segment (start 151 88.05) (end 147.05 88.05) (width 0.3048) (layer F.Cu) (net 13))
 (segment (start 147.05 88.05) (end 147 88) (width 0.3048) (layer F.Cu) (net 13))
 (segment (start 161.5 103.95) (end 165.95 103.95) (width 0.3048) (layer F.Cu) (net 11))
 (segment (start 165.95 103.95) (end 166 104) (width 0.3048) (layer F.Cu) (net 11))
 (segment (start 154 88.05) (end 154 88.5) (width 0.3048) (layer F.Cu) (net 14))
 (segment (start 149 91) (end 147.92 92.08) (width 0.3048) (layer F.Cu) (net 14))
 (segment (start 149 90) (end 149 91) (width 0.3048) (layer F.Cu) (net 14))
 (segment (start 150 89) (end 149 90) (width 0.3048) (layer F.Cu) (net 14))
 (segment (start 153.5 89) (end 150 89) (width 0.3048) (layer F.Cu) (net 14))
 (segment (start 154 88.5) (end 153.5 89) (width 0.3048) (layer F.Cu) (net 14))
 (segment (start 147.92 92.08) (end 147 92.08) (width 0.3048) (layer F.Cu) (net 14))
 (segment (start 158 103.95) (end 158 103.5) (width 0.3048) (layer F.Cu) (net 12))
 (segment (start 163.5 99.75) (end 165 99.75) (width 0.3048) (layer B.Cu) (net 12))
 (segment (start 162.75 100.5) (end 163.5 99.75) (width 0.3048) (layer B.Cu) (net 12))
 (via (at 162.75 100.5) (size 0.6) (drill 0.4) (layers F.Cu B.Cu) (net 12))
 (segment (start 163.25 101) (end 162.75 100.5) (width 0.3048) (layer F.Cu) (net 12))
 (segment (start 163.25 102.25) (end 163.25 101) (width 0.3048) (layer F.Cu) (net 12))
 (segment (start 162.5 103) (end 163.25 102.25) (width 0.3048) (layer F.Cu) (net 12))
 (segment (start 158.5 103) (end 162.5 103) (width 0.3048) (layer F.Cu) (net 12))
 (segment (start 158 103.5) (end 158.5 103) (width 0.3048) (layer F.Cu) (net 12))
 (segment (start 165 99.75) (end 166 99.92) (width 0.3048) (layer B.Cu) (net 12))
 (segment (start 158 103.95) (end 158.05 103.95) (width 0.3048) (layer F.Cu) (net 12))
 (segment (start 165.08 99.92) (end 166 99.92) (width 0.3048) (layer F.Cu) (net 12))
 (segment (start 160 88.05) (end 160 88.5) (width 0.3048) (layer F.Cu) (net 18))
 (segment (start 164.5 91.5) (end 165.08 92.08) (width 0.3048) (layer F.Cu) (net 18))
 (segment (start 164.5 89.5) (end 164.5 91.5) (width 0.3048) (layer F.Cu) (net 18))
 (segment (start 164 89) (end 164.5 89.5) (width 0.3048) (layer F.Cu) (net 18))
 (segment (start 160.5 89) (end 164 89) (width 0.3048) (layer F.Cu) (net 18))
 (segment (start 160 88.5) (end 160.5 89) (width 0.3048) (layer F.Cu) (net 18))
 (segment (start 165.08 92.08) (end 166 92.08) (width 0.3048) (layer F.Cu) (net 18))
 (segment (start 155 103.95) (end 154.95 103.95) (width 0.3048) (layer F.Cu) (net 16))
 (segment (start 154.95 103.95) (end 154 103) (width 0.3048) (layer F.Cu) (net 16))
 (segment (start 154 103) (end 149.5 103) (width 0.3048) (layer F.Cu) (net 16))
 (segment (start 149.5 103) (end 148.42 104.08) (width 0.3048) (layer F.Cu) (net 16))
 (segment (start 148.42 104.08) (end 147 104.08) (width 0.3048) (layer F.Cu) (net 16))
 (segment (start 147.3838 98.5) (end 151.25 98.5) (width 0.4064) (layer B.Cu) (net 9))
 (segment (start 164.75 97) (end 165.75 97) (width 0.4064) (layer B.Cu) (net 9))
 (segment (start 161 100.75) (end 164.75 97) (width 0.4064) (layer B.Cu) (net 9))
 (segment (start 153.5 100.75) (end 161 100.75) (width 0.4064) (layer B.Cu) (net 9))
 (segment (start 151.25 98.5) (end 153.5 100.75) (width 0.4064) (layer B.Cu) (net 9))
 (segment (start 145.75 96.5) (end 145.75 98.25) (width 0.4064) (layer B.Cu) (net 9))
 (segment (start 145.75 98.25) (end 146 98.5) (width 0.4064) (layer B.Cu) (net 9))
 (segment (start 146 98.5) (end 147.3838 98.5) (width 0.4064) (layer B.Cu) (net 9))
 (segment (start 147.3838 98.5) (end 147.3838 97.3838) (width 0.4064) (layer B.Cu) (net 9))
 (segment (start 146.5 96.5) (end 145.75 96.5) (width 0.4064) (layer B.Cu) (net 9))
 (segment (start 147.3838 97.3838) (end 146.5 96.5) (width 0.4064) (layer B.Cu) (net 9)))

